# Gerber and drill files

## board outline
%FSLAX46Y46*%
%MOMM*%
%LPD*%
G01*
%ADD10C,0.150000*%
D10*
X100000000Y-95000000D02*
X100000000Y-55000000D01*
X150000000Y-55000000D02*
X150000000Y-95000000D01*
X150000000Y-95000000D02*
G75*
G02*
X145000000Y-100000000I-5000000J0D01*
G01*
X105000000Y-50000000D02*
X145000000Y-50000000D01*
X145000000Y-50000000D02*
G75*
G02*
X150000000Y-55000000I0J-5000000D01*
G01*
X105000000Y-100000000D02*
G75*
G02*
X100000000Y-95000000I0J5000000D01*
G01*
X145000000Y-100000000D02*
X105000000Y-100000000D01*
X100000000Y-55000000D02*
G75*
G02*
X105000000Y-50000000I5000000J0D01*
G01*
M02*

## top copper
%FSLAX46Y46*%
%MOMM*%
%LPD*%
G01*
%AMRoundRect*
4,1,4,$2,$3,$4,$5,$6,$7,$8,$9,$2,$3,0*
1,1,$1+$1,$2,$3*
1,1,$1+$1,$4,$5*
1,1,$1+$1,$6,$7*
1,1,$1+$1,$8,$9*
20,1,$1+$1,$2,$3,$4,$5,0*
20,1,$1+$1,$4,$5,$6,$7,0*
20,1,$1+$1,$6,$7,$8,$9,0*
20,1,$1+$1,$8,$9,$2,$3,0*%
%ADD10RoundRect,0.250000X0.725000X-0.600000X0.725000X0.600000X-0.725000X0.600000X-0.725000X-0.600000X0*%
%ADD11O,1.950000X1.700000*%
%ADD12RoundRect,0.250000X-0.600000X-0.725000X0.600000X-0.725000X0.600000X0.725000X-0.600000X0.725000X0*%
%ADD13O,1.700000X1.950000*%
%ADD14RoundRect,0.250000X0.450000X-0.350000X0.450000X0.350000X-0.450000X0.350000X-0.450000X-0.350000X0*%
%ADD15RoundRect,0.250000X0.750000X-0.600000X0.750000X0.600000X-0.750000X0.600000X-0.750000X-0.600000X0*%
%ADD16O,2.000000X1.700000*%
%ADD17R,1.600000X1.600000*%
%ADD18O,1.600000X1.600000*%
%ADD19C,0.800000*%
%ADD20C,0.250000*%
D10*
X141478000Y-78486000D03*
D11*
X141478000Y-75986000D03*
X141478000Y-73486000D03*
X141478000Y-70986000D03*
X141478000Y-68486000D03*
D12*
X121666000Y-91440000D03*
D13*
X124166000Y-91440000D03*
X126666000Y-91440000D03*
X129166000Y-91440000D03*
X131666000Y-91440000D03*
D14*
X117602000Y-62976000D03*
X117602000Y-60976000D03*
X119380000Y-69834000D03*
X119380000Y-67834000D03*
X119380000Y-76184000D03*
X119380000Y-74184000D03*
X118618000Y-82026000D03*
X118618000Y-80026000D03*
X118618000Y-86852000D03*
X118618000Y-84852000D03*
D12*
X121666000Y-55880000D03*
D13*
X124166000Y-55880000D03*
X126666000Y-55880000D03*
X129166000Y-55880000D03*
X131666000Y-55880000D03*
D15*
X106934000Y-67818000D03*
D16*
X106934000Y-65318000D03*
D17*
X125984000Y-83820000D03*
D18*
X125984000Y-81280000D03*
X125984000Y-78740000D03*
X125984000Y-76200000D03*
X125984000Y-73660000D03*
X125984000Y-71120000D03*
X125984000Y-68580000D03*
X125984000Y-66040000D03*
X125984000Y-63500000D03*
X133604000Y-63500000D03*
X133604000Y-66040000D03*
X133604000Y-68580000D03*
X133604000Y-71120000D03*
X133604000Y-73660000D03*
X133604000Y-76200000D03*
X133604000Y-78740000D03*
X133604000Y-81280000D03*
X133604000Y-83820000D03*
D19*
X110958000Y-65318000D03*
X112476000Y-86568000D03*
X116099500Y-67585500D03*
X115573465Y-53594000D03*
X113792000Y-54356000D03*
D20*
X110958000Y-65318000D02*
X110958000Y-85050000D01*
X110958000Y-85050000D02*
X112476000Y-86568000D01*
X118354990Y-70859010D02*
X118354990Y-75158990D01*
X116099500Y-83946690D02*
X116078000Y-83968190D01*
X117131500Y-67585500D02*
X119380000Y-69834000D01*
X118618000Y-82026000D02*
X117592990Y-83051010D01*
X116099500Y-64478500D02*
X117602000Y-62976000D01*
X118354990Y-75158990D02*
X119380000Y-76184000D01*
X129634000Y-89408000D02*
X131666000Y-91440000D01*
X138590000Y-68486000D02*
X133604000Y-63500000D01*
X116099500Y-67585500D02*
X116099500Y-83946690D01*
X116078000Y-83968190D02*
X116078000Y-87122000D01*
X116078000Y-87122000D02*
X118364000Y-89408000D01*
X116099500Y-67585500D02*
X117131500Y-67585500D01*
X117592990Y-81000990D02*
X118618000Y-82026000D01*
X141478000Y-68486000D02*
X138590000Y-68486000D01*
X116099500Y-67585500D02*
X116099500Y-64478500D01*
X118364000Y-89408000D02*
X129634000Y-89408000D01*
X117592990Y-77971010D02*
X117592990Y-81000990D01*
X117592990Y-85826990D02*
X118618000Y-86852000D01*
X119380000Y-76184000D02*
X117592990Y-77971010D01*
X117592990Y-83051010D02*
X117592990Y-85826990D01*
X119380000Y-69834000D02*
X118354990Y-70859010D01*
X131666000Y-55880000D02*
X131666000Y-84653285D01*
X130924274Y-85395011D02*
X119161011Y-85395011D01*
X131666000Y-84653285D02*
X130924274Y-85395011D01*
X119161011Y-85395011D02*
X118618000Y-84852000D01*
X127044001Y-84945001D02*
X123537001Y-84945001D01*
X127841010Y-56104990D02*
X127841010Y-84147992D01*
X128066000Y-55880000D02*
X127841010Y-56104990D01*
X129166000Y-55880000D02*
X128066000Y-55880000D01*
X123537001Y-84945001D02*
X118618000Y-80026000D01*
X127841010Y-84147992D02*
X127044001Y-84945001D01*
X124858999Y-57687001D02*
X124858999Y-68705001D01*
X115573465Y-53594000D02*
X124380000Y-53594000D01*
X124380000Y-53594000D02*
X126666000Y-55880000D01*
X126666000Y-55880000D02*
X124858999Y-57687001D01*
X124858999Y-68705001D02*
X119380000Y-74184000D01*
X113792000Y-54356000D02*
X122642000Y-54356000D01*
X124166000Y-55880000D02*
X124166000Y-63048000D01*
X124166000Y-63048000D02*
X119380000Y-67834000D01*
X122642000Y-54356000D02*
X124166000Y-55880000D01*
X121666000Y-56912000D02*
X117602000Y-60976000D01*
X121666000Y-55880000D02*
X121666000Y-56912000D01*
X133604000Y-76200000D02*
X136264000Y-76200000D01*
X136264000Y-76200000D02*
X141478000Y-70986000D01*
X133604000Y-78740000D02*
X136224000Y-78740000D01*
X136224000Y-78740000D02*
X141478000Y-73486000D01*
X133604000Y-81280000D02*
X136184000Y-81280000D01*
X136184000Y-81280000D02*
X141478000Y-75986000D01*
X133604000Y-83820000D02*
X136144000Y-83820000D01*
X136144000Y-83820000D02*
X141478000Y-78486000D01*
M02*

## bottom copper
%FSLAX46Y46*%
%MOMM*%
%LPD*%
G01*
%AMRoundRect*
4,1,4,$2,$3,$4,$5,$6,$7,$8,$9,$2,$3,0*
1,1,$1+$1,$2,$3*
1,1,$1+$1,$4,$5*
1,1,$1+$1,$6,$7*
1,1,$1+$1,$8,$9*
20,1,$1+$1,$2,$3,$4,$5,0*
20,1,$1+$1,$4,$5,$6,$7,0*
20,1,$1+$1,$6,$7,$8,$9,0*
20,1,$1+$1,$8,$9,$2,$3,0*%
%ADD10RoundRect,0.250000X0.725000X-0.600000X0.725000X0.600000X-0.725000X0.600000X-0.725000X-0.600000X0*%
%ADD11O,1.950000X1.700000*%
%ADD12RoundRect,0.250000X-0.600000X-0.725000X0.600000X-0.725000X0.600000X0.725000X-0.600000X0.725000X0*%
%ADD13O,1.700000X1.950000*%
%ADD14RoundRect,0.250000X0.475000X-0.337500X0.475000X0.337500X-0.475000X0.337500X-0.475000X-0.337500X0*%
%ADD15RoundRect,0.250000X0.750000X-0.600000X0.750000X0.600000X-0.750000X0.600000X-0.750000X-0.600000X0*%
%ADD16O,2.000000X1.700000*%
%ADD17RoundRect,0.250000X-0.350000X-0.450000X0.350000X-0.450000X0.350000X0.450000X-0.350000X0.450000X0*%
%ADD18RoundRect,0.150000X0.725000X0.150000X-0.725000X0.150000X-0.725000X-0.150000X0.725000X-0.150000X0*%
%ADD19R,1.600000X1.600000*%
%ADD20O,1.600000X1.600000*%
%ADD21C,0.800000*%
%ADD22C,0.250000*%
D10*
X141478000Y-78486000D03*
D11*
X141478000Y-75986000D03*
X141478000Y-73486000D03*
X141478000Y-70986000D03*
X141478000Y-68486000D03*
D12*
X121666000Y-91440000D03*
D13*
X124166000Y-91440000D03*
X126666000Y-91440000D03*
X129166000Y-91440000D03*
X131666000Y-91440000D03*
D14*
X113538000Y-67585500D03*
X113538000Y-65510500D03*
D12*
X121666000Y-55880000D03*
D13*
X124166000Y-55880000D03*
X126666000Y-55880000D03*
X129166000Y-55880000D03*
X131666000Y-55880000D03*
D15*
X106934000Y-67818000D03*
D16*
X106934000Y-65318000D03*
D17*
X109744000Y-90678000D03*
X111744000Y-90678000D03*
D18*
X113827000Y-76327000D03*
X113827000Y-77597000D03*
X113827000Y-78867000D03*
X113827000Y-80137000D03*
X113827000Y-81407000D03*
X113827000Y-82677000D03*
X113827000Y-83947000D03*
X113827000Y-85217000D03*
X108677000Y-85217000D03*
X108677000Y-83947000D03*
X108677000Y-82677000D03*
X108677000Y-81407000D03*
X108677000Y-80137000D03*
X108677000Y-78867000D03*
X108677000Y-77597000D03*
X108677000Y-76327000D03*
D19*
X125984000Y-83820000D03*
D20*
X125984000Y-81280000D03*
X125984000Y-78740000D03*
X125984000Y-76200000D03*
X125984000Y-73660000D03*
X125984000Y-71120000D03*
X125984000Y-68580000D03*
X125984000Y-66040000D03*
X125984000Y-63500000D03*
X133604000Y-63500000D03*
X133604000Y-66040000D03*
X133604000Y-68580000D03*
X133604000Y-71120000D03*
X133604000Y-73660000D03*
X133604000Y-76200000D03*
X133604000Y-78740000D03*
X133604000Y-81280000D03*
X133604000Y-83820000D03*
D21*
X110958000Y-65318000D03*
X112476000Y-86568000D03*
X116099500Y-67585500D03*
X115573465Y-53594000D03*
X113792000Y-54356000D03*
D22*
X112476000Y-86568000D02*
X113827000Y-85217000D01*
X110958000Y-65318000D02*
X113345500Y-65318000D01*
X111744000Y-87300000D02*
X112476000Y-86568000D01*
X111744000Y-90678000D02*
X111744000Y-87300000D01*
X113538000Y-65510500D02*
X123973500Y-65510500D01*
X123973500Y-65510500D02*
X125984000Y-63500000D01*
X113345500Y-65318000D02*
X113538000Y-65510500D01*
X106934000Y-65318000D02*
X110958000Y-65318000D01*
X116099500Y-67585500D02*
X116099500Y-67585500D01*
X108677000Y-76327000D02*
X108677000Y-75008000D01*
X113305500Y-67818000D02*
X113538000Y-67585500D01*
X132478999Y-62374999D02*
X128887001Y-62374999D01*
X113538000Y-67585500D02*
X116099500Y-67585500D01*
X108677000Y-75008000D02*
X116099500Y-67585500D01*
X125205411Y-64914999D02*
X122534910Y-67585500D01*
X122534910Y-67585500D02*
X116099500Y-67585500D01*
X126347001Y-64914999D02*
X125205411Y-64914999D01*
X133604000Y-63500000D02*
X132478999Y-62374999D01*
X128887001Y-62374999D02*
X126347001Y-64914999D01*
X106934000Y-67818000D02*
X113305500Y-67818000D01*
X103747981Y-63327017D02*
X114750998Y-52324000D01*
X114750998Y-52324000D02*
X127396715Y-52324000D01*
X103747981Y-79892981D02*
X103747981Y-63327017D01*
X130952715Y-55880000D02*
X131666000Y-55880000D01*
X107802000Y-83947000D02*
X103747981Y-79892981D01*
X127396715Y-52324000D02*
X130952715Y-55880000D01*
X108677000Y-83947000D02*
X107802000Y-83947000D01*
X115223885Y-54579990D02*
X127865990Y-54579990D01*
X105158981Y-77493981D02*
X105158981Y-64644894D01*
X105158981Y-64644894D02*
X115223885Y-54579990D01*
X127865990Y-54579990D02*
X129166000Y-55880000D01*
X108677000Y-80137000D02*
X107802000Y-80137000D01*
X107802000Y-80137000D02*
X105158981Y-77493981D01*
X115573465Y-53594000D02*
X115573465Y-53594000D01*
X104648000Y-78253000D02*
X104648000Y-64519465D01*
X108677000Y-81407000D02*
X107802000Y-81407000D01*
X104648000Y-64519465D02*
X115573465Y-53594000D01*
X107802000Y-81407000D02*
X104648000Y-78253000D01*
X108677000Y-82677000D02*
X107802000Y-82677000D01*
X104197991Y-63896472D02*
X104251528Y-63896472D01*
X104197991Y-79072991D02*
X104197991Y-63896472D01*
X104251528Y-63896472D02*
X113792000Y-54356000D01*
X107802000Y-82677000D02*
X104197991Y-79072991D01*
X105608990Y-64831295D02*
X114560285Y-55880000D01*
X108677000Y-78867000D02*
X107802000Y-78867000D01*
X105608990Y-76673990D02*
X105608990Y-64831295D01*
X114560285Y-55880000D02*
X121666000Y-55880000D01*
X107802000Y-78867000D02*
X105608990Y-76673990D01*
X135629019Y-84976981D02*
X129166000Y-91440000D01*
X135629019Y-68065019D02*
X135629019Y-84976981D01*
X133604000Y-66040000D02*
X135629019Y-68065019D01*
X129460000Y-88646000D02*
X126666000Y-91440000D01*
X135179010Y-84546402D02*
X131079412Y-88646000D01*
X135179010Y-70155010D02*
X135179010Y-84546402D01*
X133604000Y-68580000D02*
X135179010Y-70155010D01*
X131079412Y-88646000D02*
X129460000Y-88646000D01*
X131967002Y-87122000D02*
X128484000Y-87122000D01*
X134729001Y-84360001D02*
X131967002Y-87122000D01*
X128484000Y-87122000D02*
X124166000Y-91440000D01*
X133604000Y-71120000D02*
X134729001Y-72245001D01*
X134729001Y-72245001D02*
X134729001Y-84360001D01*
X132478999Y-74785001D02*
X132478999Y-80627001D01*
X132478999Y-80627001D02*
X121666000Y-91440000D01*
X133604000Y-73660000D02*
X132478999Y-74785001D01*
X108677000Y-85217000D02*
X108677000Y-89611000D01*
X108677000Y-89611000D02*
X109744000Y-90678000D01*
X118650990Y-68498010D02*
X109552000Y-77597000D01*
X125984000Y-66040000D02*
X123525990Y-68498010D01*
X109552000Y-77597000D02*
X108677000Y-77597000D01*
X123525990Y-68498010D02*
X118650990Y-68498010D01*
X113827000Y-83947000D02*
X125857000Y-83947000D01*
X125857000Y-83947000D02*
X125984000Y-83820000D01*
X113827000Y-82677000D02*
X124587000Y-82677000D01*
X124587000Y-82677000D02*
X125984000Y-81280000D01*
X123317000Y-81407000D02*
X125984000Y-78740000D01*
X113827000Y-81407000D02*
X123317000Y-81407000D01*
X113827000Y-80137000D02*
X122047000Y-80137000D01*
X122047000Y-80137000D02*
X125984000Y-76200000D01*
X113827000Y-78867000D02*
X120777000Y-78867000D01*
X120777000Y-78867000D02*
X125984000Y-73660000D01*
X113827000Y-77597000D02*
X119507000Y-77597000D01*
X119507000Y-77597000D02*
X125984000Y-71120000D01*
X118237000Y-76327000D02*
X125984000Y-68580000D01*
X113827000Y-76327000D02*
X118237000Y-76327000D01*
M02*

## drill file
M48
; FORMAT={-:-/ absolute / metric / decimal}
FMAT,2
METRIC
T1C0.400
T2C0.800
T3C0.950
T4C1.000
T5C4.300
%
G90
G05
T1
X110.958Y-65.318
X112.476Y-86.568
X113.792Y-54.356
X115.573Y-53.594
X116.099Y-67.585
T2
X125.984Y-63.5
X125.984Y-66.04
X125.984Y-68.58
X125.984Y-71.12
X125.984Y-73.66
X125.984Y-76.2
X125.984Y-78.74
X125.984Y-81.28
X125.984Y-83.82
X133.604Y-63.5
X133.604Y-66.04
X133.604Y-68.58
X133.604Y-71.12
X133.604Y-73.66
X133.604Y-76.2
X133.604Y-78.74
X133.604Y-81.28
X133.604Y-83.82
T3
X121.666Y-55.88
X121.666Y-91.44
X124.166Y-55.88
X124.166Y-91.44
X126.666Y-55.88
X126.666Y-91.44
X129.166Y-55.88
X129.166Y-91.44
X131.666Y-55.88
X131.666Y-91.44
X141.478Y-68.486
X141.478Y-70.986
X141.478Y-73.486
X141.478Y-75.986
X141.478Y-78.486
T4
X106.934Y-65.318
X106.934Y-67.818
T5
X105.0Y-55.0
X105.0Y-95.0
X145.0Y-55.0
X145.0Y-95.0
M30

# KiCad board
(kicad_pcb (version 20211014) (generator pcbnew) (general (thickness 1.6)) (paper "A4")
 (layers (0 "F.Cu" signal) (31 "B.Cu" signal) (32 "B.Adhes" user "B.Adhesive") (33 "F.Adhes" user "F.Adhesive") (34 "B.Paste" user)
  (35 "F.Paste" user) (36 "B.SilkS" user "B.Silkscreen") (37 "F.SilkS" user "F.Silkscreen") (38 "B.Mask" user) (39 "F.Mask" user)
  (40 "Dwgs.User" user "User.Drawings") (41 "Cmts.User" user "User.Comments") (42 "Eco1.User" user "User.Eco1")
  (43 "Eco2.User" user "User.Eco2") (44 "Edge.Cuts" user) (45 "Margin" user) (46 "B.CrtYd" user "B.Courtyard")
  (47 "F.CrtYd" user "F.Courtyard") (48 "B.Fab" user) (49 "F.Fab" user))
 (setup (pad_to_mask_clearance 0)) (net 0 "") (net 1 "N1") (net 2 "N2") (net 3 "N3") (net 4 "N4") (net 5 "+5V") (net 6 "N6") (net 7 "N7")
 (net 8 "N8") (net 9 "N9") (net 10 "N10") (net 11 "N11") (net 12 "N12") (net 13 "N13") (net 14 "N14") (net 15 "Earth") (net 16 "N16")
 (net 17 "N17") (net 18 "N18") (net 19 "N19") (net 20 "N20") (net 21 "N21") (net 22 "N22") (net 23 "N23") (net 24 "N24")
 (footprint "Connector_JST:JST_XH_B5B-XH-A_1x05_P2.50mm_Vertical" (layer "F.Cu") (at 141.478 78.486 90)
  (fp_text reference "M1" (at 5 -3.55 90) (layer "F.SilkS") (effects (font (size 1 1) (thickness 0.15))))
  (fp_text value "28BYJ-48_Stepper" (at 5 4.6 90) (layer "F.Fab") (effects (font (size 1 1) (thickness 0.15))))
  (pad "1" thru_hole roundrect locked (at 0 0 90) (size 1.7 1.95) (drill 0.95) (layers *.Cu *.Mask) (roundrect_rratio 0.147059) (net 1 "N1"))
  (pad "2" thru_hole oval locked (at 2.5 0 90) (size 1.7 1.95) (drill 0.95) (layers *.Cu *.Mask) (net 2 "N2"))
  (pad "3" thru_hole oval locked (at 5 0 90) (size 1.7 1.95) (drill 0.95) (layers *.Cu *.Mask) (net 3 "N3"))
  (pad "4" thru_hole oval locked (at 7.5 0 90) (size 1.7 1.95) (drill 0.95) (layers *.Cu *.Mask) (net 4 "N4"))
  (pad "5" thru_hole oval locked (at 10 0 90) (size 1.7 1.95) (drill 0.95) (layers *.Cu *.Mask) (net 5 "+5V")))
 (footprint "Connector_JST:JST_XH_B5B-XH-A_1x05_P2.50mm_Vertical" (layer "F.Cu") (at 121.666 91.44)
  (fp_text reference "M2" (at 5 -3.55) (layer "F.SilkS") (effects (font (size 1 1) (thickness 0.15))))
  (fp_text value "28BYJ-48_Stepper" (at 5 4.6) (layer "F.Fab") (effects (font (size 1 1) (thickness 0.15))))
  (pad "1" thru_hole roundrect locked (at 0 0) (size 1.7 1.95) (drill 0.95) (layers *.Cu *.Mask) (roundrect_rratio 0.147059) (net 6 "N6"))
  (pad "2" thru_hole oval locked (at 2.5 0) (size 1.7 1.95) (drill 0.95) (layers *.Cu *.Mask) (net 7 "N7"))
  (pad "3" thru_hole oval locked (at 5 0) (size 1.7 1.95) (drill 0.95) (layers *.Cu *.Mask) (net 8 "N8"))
  (pad "4" thru_hole oval locked (at 7.5 0) (size 1.7 1.95) (drill 0.95) (layers *.Cu *.Mask) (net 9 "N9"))
  (pad "5" thru_hole oval locked (at 10 0) (size 1.7 1.95) (drill 0.95) (layers *.Cu *.Mask) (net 5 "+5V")))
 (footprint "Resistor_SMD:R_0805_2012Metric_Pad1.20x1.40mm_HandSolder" (layer "F.Cu") (at 117.602 61.976 90)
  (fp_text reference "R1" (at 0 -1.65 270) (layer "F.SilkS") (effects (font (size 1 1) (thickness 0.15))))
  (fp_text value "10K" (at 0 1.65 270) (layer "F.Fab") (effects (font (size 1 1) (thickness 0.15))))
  (pad "1" smd roundrect locked (at -1 0 90) (size 1.2 1.4) (layers "F.Cu" "F.Paste" "F.Mask") (roundrect_rratio 0.208333) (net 5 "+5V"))
  (pad "2" smd roundrect locked (at 1 0 90) (size 1.2 1.4) (layers "F.Cu" "F.Paste" "F.Mask") (roundrect_rratio 0.208333) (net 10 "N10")))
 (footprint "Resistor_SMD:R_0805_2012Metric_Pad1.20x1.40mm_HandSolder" (layer "F.Cu") (at 119.38 68.834 90)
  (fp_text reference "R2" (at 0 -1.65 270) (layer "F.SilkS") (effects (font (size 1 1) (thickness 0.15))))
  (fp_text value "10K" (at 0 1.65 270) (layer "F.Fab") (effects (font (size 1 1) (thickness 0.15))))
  (pad "1" smd roundrect locked (at -1 0 90) (size 1.2 1.4) (layers "F.Cu" "F.Paste" "F.Mask") (roundrect_rratio 0.208333) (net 5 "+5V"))
  (pad "2" smd roundrect locked (at 1 0 90) (size 1.2 1.4) (layers "F.Cu" "F.Paste" "F.Mask") (roundrect_rratio 0.208333) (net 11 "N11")))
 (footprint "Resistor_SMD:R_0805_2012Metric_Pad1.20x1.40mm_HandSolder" (layer "F.Cu") (at 119.38 75.184 90)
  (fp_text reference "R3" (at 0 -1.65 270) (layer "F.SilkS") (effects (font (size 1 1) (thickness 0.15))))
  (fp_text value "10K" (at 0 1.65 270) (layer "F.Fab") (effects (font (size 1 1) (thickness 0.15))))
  (pad "1" smd roundrect locked (at -1 0 90) (size 1.2 1.4) (layers "F.Cu" "F.Paste" "F.Mask") (roundrect_rratio 0.208333) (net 5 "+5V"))
  (pad "2" smd roundrect locked (at 1 0 90) (size 1.2 1.4) (layers "F.Cu" "F.Paste" "F.Mask") (roundrect_rratio 0.208333) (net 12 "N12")))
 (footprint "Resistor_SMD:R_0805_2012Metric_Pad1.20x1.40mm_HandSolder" (layer "F.Cu") (at 118.618 81.026 90)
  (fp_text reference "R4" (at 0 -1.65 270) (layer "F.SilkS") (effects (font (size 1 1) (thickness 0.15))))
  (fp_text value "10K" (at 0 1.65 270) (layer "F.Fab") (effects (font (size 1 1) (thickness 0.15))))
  (pad "1" smd roundrect locked (at -1 0 90) (size 1.2 1.4) (layers "F.Cu" "F.Paste" "F.Mask") (roundrect_rratio 0.208333) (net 5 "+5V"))
  (pad "2" smd roundrect locked (at 1 0 90) (size 1.2 1.4) (layers "F.Cu" "F.Paste" "F.Mask") (roundrect_rratio 0.208333) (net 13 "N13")))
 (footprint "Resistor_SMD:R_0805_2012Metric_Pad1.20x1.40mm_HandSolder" (layer "F.Cu") (at 118.618 85.852 90)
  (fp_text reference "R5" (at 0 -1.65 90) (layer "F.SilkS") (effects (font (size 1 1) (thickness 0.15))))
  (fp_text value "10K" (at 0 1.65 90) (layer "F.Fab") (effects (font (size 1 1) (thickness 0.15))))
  (pad "1" smd roundrect locked (at -1 0 90) (size 1.2 1.4) (layers "F.Cu" "F.Paste" "F.Mask") (roundrect_rratio 0.208333) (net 5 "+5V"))
  (pad "2" smd roundrect locked (at 1 0 90) (size 1.2 1.4) (layers "F.Cu" "F.Paste" "F.Mask") (roundrect_rratio 0.208333) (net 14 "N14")))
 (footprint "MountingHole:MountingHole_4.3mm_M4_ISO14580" (layer "F.Cu") (at 105 55)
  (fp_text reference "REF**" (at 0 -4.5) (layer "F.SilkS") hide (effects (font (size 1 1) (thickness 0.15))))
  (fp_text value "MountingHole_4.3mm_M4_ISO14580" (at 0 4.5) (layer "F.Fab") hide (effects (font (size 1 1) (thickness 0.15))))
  (pad "" np_thru_hole circle locked (at 0 0) (size 4.3 4.3) (drill 4.3) (layers *.Cu *.Mask)))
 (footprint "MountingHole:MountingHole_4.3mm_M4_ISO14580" (layer "F.Cu") (at 145 55)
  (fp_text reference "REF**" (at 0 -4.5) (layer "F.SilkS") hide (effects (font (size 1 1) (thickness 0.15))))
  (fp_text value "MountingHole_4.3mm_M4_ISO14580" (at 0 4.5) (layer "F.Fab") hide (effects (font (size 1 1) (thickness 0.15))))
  (pad "" np_thru_hole circle locked (at 0 0) (size 4.3 4.3) (drill 4.3) (layers *.Cu *.Mask)))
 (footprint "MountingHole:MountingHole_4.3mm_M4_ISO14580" (layer "F.Cu") (at 105 95)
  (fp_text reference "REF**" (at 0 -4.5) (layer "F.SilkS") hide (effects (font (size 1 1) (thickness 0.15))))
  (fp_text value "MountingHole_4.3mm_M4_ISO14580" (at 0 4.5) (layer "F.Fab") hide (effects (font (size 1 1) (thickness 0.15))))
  (pad "" np_thru_hole circle locked (at 0 0) (size 4.3 4.3) (drill 4.3) (layers *.Cu *.Mask)))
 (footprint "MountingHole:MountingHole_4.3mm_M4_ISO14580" (layer "F.Cu") (at 145 95)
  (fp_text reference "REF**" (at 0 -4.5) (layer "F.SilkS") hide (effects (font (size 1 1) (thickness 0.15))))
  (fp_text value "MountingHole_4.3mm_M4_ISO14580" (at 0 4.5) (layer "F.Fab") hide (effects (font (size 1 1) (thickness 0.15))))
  (pad "" np_thru_hole circle locked (at 0 0) (size 4.3 4.3) (drill 4.3) (layers *.Cu *.Mask)))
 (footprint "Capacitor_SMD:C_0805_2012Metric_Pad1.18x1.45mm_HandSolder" (layer "B.Cu") (at 113.538 66.548 90)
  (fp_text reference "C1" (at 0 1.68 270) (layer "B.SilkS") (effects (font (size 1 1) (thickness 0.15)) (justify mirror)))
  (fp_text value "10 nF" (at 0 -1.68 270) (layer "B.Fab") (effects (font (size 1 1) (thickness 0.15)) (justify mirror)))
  (pad "1" smd roundrect locked (at -1.0375 0 90) (size 1.175 1.45) (layers "B.Cu" "B.Paste" "B.Mask") (roundrect_rratio 0.212766)
   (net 5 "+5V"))
  (pad "2" smd roundrect locked (at 1.0375 0 90) (size 1.175 1.45) (layers "B.Cu" "B.Paste" "B.Mask") (roundrect_rratio 0.212766)
   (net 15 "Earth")))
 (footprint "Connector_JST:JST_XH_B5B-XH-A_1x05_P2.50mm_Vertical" (layer "B.Cu") (at 121.666 55.88)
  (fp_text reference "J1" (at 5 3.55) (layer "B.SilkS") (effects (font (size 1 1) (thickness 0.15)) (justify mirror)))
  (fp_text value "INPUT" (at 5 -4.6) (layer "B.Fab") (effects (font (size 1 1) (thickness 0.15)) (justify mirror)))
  (pad "1" thru_hole roundrect locked (at 0 0) (size 1.7 1.95) (drill 0.95) (layers *.Cu *.Mask) (roundrect_rratio 0.147059) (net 10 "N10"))
  (pad "2" thru_hole oval locked (at 2.5 0) (size 1.7 1.95) (drill 0.95) (layers *.Cu *.Mask) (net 11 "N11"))
  (pad "3" thru_hole oval locked (at 5 0) (size 1.7 1.95) (drill 0.95) (layers *.Cu *.Mask) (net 12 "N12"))
  (pad "4" thru_hole oval locked (at 7.5 0) (size 1.7 1.95) (drill 0.95) (layers *.Cu *.Mask) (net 13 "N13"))
  (pad "5" thru_hole oval locked (at 10 0) (size 1.7 1.95) (drill 0.95) (layers *.Cu *.Mask) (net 14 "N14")))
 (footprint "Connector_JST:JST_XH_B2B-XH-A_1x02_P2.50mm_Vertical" (layer "B.Cu") (at 106.934 67.818 90)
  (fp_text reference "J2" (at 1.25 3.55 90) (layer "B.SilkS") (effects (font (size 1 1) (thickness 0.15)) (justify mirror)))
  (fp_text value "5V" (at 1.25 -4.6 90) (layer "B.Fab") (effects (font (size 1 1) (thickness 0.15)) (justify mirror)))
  (pad "1" thru_hole roundrect locked (at 0 0 90) (size 1.7 2) (drill 1) (layers *.Cu *.Mask) (roundrect_rratio 0.147059) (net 5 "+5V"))
  (pad "2" thru_hole oval locked (at 2.5 0 90) (size 1.7 2) (drill 1) (layers *.Cu *.Mask) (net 15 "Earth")))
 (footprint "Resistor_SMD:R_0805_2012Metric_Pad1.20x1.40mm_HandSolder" (layer "B.Cu") (at 110.744 90.678)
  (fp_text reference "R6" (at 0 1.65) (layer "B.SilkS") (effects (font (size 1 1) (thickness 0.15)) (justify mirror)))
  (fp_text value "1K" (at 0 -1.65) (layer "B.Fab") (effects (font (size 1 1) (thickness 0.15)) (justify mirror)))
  (pad "1" smd roundrect locked (at -1 0) (size 1.2 1.4) (layers "B.Cu" "B.Paste" "B.Mask") (roundrect_rratio 0.208333) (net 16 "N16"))
  (pad "2" smd roundrect locked (at 1 0) (size 1.2 1.4) (layers "B.Cu" "B.Paste" "B.Mask") (roundrect_rratio 0.208333) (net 15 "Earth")))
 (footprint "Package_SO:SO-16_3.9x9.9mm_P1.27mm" (layer "B.Cu") (at 111.252 80.772 180)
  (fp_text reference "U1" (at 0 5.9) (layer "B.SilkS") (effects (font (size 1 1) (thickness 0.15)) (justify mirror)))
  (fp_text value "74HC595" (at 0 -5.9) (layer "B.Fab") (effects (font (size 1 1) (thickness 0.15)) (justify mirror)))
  (pad "1" smd roundrect locked (at -2.575 4.445 180) (size 1.75 0.6) (layers "B.Cu" "B.Paste" "B.Mask") (roundrect_rratio 0.25)
   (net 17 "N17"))
  (pad "2" smd roundrect locked (at -2.575 3.175 180) (size 1.75 0.6) (layers "B.Cu" "B.Paste" "B.Mask") (roundrect_rratio 0.25)
   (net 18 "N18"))
  (pad "3" smd roundrect locked (at -2.575 1.905 180) (size 1.75 0.6) (layers "B.Cu" "B.Paste" "B.Mask") (roundrect_rratio 0.25)
   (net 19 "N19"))
  (pad "4" smd roundrect locked (at -2.575 0.635 180) (size 1.75 0.6) (layers "B.Cu" "B.Paste" "B.Mask") (roundrect_rratio 0.25)
   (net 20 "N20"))
  (pad "5" smd roundrect locked (at -2.575 -0.635 180) (size 1.75 0.6) (layers "B.Cu" "B.Paste" "B.Mask") (roundrect_rratio 0.25)
   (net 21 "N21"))
  (pad "6" smd roundrect locked (at -2.575 -1.905 180) (size 1.75 0.6) (layers "B.Cu" "B.Paste" "B.Mask") (roundrect_rratio 0.25)
   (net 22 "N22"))
  (pad "7" smd roundrect locked (at -2.575 -3.175 180) (size 1.75 0.6) (layers "B.Cu" "B.Paste" "B.Mask") (roundrect_rratio 0.25)
   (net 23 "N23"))
  (pad "8" smd roundrect locked (at -2.575 -4.445 180) (size 1.75 0.6) (layers "B.Cu" "B.Paste" "B.Mask") (roundrect_rratio 0.25)
   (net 15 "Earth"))
  (pad "9" smd roundrect locked (at 2.575 -4.445 180) (size 1.75 0.6) (layers "B.Cu" "B.Paste" "B.Mask") (roundrect_rratio 0.25)
   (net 16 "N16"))
  (pad "10" smd roundrect locked (at 2.575 -3.175 180) (size 1.75 0.6) (layers "B.Cu" "B.Paste" "B.Mask") (roundrect_rratio 0.25)
   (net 14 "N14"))
  (pad "11" smd roundrect locked (at 2.575 -1.905 180) (size 1.75 0.6) (layers "B.Cu" "B.Paste" "B.Mask") (roundrect_rratio 0.25)
   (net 11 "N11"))
  (pad "12" smd roundrect locked (at 2.575 -0.635 180) (size 1.75 0.6) (layers "B.Cu" "B.Paste" "B.Mask") (roundrect_rratio 0.25)
   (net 12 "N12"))
  (pad "13" smd roundrect locked (at 2.575 0.635 180) (size 1.75 0.6) (layers "B.Cu" "B.Paste" "B.Mask") (roundrect_rratio 0.25)
   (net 13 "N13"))
  (pad "14" smd roundrect locked (at 2.575 1.905 180) (size 1.75 0.6) (layers "B.Cu" "B.Paste" "B.Mask") (roundrect_rratio 0.25)
   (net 10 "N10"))
  (pad "15" smd roundrect locked (at 2.575 3.175 180) (size 1.75 0.6) (layers "B.Cu" "B.Paste" "B.Mask") (roundrect_rratio 0.25)
   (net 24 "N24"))
  (pad "16" smd roundrect locked (at 2.575 4.445 180) (size 1.75 0.6) (layers "B.Cu" "B.Paste" "B.Mask") (roundrect_rratio 0.25)
   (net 5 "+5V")))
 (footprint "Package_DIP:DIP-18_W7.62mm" (layer "B.Cu") (at 125.984 83.82)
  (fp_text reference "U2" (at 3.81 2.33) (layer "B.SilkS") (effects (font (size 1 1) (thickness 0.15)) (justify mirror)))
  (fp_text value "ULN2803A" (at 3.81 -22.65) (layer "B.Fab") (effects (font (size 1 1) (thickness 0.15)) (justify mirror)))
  (pad "1" thru_hole rect locked (at 0 0) (size 1.6 1.6) (drill 0.8) (layers *.Cu *.Mask) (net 23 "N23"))
  (pad "2" thru_hole oval locked (at 0 -2.54) (size 1.6 1.6) (drill 0.8) (layers *.Cu *.Mask) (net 22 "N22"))
  (pad "3" thru_hole oval locked (at 0 -5.08) (size 1.6 1.6) (drill 0.8) (layers *.Cu *.Mask) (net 21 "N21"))
  (pad "4" thru_hole oval locked (at 0 -7.62) (size 1.6 1.6) (drill 0.8) (layers *.Cu *.Mask) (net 20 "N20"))
  (pad "5" thru_hole oval locked (at 0 -10.16) (size 1.6 1.6) (drill 0.8) (layers *.Cu *.Mask) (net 19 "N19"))
  (pad "6" thru_hole oval locked (at 0 -12.7) (size 1.6 1.6) (drill 0.8) (layers *.Cu *.Mask) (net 18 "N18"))
  (pad "7" thru_hole oval locked (at 0 -15.24) (size 1.6 1.6) (drill 0.8) (layers *.Cu *.Mask) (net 17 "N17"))
  (pad "8" thru_hole oval locked (at 0 -17.78) (size 1.6 1.6) (drill 0.8) (layers *.Cu *.Mask) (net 24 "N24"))
  (pad "9" thru_hole oval locked (at 0 -20.32) (size 1.6 1.6) (drill 0.8) (layers *.Cu *.Mask) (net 15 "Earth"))
  (pad "10" thru_hole oval locked (at 7.62 -20.32) (size 1.6 1.6) (drill 0.8) (layers *.Cu *.Mask) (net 5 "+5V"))
  (pad "11" thru_hole oval locked (at 7.62 -17.78) (size 1.6 1.6) (drill 0.8) (layers *.Cu *.Mask) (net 9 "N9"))
  (pad "12" thru_hole oval locked (at 7.62 -15.24) (size 1.6 1.6) (drill 0.8) (layers *.Cu *.Mask) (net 8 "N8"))
  (pad "13" thru_hole oval locked (at 7.62 -12.7) (size 1.6 1.6) (drill 0.8) (layers *.Cu *.Mask) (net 7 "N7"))
  (pad "14" thru_hole oval locked (at 7.62 -10.16) (size 1.6 1.6) (drill 0.8) (layers *.Cu *.Mask) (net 6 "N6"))
  (pad "15" thru_hole oval locked (at 7.62 -7.62) (size 1.6 1.6) (drill 0.8) (layers *.Cu *.Mask) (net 4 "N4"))
  (pad "16" thru_hole oval locked (at 7.62 -5.08) (size 1.6 1.6) (drill 0.8) (layers *.Cu *.Mask) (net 3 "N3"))
  (pad "17" thru_hole oval locked (at 7.62 -2.54) (size 1.6 1.6) (drill 0.8) (layers *.Cu *.Mask) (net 2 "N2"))
  (pad "18" thru_hole oval locked (at 7.62 0) (size 1.6 1.6) (drill 0.8) (layers *.Cu *.Mask) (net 1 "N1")))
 (gr_line (start 100 95) (end 100 55) (layer "Edge.Cuts") (width 0.15))
 (gr_line (start 150 55) (end 150 95) (layer "Edge.Cuts") (width 0.15))
 (gr_arc (start 150 95) (mid 148.535534 98.535534) (end 145 100) (layer "Edge.Cuts") (width 0.15))
 (gr_line (start 105 50) (end 145 50) (layer "Edge.Cuts") (width 0.15))
 (gr_arc (start 145 50) (mid 148.535534 51.464466) (end 150 55) (layer "Edge.Cuts") (width 0.15))
 (gr_arc (start 105 100) (mid 101.464466 98.535534) (end 100 95) (layer "Edge.Cuts") (width 0.15))
 (gr_line (start 145 100) (end 105 100) (layer "Edge.Cuts") (width 0.15))
 (gr_arc (start 100 55) (mid 101.464466 51.464466) (end 105 50) (layer "Edge.Cuts") (width 0.15))
 (segment (start 110.958 65.318) (end 110.958 85.05) (width 0.25) (layer "F.Cu") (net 15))
 (segment (start 110.958 85.05) (end 112.476 86.568) (width 0.25) (layer "F.Cu") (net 15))
 (via (at 110.958 65.318) (size 0.8) (drill 0.4) (layers "F.Cu" "B.Cu") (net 15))
 (via (at 112.476 86.568) (size 0.8) (drill 0.4) (layers "F.Cu" "B.Cu") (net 15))
 (segment (start 112.476 86.568) (end 113.827 85.217) (width 0.25) (layer "B.Cu") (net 15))
 (segment (start 110.958 65.318) (end 113.3455 65.318) (width 0.25) (layer "B.Cu") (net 15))
 (segment (start 111.744 87.3) (end 112.476 86.568) (width 0.25) (layer "B.Cu") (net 15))
 (segment (start 111.744 90.678) (end 111.744 87.3) (width 0.25) (layer "B.Cu") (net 15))
 (segment (start 113.538 65.5105) (end 123.9735 65.5105) (width 0.25) (layer "B.Cu") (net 15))
 (segment (start 123.9735 65.5105) (end 125.984 63.5) (width 0.25) (layer "B.Cu") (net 15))
 (segment (start 113.3455 65.318) (end 113.538 65.5105) (width 0.25) (layer "B.Cu") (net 15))
 (segment (start 106.934 65.318) (end 110.958 65.318) (width 0.25) (layer "B.Cu") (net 15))
 (segment (start 118.35499 70.85901) (end 118.35499 75.15899) (width 0.25) (layer "F.Cu") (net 5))
 (segment (start 116.0995 83.94669) (end 116.078 83.96819) (width 0.25) (layer "F.Cu") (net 5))
 (segment (start 117.1315 67.5855) (end 119.38 69.834) (width 0.25) (layer "F.Cu") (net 5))
 (segment (start 118.618 82.026) (end 117.59299 83.05101) (width 0.25) (layer "F.Cu") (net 5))
 (segment (start 116.0995 64.4785) (end 117.602 62.976) (width 0.25) (layer "F.Cu") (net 5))
 (segment (start 118.35499 75.15899) (end 119.38 76.184) (width 0.25) (layer "F.Cu") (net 5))
 (segment (start 129.634 89.408) (end 131.666 91.44) (width 0.25) (layer "F.Cu") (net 5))
 (segment (start 138.59 68.486) (end 133.604 63.5) (width 0.25) (layer "F.Cu") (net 5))
 (segment (start 116.0995 67.5855) (end 116.0995 83.94669) (width 0.25) (layer "F.Cu") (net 5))
 (segment (start 116.078 83.96819) (end 116.078 87.122) (width 0.25) (layer "F.Cu") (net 5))
 (segment (start 116.078 87.122) (end 118.364 89.408) (width 0.25) (layer "F.Cu") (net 5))
 (segment (start 116.0995 67.5855) (end 117.1315 67.5855) (width 0.25) (layer "F.Cu") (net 5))
 (segment (start 117.59299 81.00099) (end 118.618 82.026) (width 0.25) (layer "F.Cu") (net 5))
 (segment (start 141.478 68.486) (end 138.59 68.486) (width 0.25) (layer "F.Cu") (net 5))
 (segment (start 116.0995 67.5855) (end 116.0995 64.4785) (width 0.25) (layer "F.Cu") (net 5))
 (segment (start 118.364 89.408) (end 129.634 89.408) (width 0.25) (layer "F.Cu") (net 5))
 (segment (start 117.59299 77.97101) (end 117.59299 81.00099) (width 0.25) (layer "F.Cu") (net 5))
 (segment (start 117.59299 85.82699) (end 118.618 86.852) (width 0.25) (layer "F.Cu") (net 5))
 (segment (start 119.38 76.184) (end 117.59299 77.97101) (width 0.25) (layer "F.Cu") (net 5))
 (segment (start 117.59299 83.05101) (end 117.59299 85.82699) (width 0.25) (layer "F.Cu") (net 5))
 (segment (start 119.38 69.834) (end 118.35499 70.85901) (width 0.25) (layer "F.Cu") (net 5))
 (via (at 116.0995 67.5855) (size 0.8) (drill 0.4) (layers "F.Cu" "B.Cu") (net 5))
 (segment (start 116.0995 67.5855) (end 116.0995 67.5855) (width 0.25) (layer "B.Cu") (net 5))
 (segment (start 108.677 76.327) (end 108.677 75.008) (width 0.25) (layer "B.Cu") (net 5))
 (segment (start 113.3055 67.818) (end 113.538 67.5855) (width 0.25) (layer "B.Cu") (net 5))
 (segment (start 132.478999 62.374999) (end 128.887001 62.374999) (width 0.25) (layer "B.Cu") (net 5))
 (segment (start 113.538 67.5855) (end 116.0995 67.5855) (width 0.25) (layer "B.Cu") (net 5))
 (segment (start 108.677 75.008) (end 116.0995 67.5855) (width 0.25) (layer "B.Cu") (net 5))
 (segment (start 125.205411 64.914999) (end 122.53491 67.5855) (width 0.25) (layer "B.Cu") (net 5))
 (segment (start 122.53491 67.5855) (end 116.0995 67.5855) (width 0.25) (layer "B.Cu") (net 5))
 (segment (start 126.347001 64.914999) (end 125.205411 64.914999) (width 0.25) (layer "B.Cu") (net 5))
 (segment (start 133.604 63.5) (end 132.478999 62.374999) (width 0.25) (layer "B.Cu") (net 5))
 (segment (start 128.887001 62.374999) (end 126.347001 64.914999) (width 0.25) (layer "B.Cu") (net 5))
 (segment (start 106.934 67.818) (end 113.3055 67.818) (width 0.25) (layer "B.Cu") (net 5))
 (segment (start 131.666 55.88) (end 131.666 84.653285) (width 0.25) (layer "F.Cu") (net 14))
 (segment (start 130.924274 85.395011) (end 119.161011 85.395011) (width 0.25) (layer "F.Cu") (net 14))
 (segment (start 131.666 84.653285) (end 130.924274 85.395011) (width 0.25) (layer "F.Cu") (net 14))
 (segment (start 119.161011 85.395011) (end 118.618 84.852) (width 0.25) (layer "F.Cu") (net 14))
 (segment (start 103.747981 63.327017) (end 114.750998 52.324) (width 0.25) (layer "B.Cu") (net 14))
 (segment (start 114.750998 52.324) (end 127.396715 52.324) (width 0.25) (layer "B.Cu") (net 14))
 (segment (start 103.747981 79.892981) (end 103.747981 63.327017) (width 0.25) (layer "B.Cu") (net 14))
 (segment (start 130.952715 55.88) (end 131.666 55.88) (width 0.25) (layer "B.Cu") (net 14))
 (segment (start 107.802 83.947) (end 103.747981 79.892981) (width 0.25) (layer "B.Cu") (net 14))
 (segment (start 127.396715 52.324) (end 130.952715 55.88) (width 0.25) (layer "B.Cu") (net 14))
 (segment (start 108.677 83.947) (end 107.802 83.947) (width 0.25) (layer "B.Cu") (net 14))
 (segment (start 127.044001 84.945001) (end 123.537001 84.945001) (width 0.25) (layer "F.Cu") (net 13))
 (segment (start 127.84101 56.10499) (end 127.84101 84.147992) (width 0.25) (layer "F.Cu") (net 13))
 (segment (start 128.066 55.88) (end 127.84101 56.10499) (width 0.25) (layer "F.Cu") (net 13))
 (segment (start 129.166 55.88) (end 128.066 55.88) (width 0.25) (layer "F.Cu") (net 13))
 (segment (start 123.537001 84.945001) (end 118.618 80.026) (width 0.25) (layer "F.Cu") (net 13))
 (segment (start 127.84101 84.147992) (end 127.044001 84.945001) (width 0.25) (layer "F.Cu") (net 13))
 (segment (start 115.223885 54.57999) (end 127.86599 54.57999) (width 0.25) (layer "B.Cu") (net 13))
 (segment (start 105.158981 77.493981) (end 105.158981 64.644894) (width 0.25) (layer "B.Cu") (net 13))
 (segment (start 105.158981 64.644894) (end 115.223885 54.57999) (width 0.25) (layer "B.Cu") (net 13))
 (segment (start 127.86599 54.57999) (end 129.166 55.88) (width 0.25) (layer "B.Cu") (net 13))
 (segment (start 108.677 80.137) (end 107.802 80.137) (width 0.25) (layer "B.Cu") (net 13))
 (segment (start 107.802 80.137) (end 105.158981 77.493981) (width 0.25) (layer "B.Cu") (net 13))
 (segment (start 124.858999 57.687001) (end 124.858999 68.705001) (width 0.25) (layer "F.Cu") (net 12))
 (segment (start 115.573465 53.594) (end 124.38 53.594) (width 0.25) (layer "F.Cu") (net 12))
 (segment (start 124.38 53.594) (end 126.666 55.88) (width 0.25) (layer "F.Cu") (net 12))
 (segment (start 126.666 55.88) (end 124.858999 57.687001) (width 0.25) (layer "F.Cu") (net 12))
 (segment (start 124.858999 68.705001) (end 119.38 74.184) (width 0.25) (layer "F.Cu") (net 12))
 (via (at 115.573465 53.594) (size 0.8) (drill 0.4) (layers "F.Cu" "B.Cu") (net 12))
 (segment (start 115.573465 53.594) (end 115.573465 53.594) (width 0.25) (layer "B.Cu") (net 12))
 (segment (start 104.648 78.253) (end 104.648 64.519465) (width 0.25) (layer "B.Cu") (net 12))
 (segment (start 108.677 81.407) (end 107.802 81.407) (width 0.25) (layer "B.Cu") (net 12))
 (segment (start 104.648 64.519465) (end 115.573465 53.594) (width 0.25) (layer "B.Cu") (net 12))
 (segment (start 107.802 81.407) (end 104.648 78.253) (width 0.25) (layer "B.Cu") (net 12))
 (segment (start 113.792 54.356) (end 122.642 54.356) (width 0.25) (layer "F.Cu") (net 11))
 (segment (start 124.166 55.88) (end 124.166 63.048) (width 0.25) (layer "F.Cu") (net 11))
 (segment (start 124.166 63.048) (end 119.38 67.834) (width 0.25) (layer "F.Cu") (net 11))
 (segment (start 122.642 54.356) (end 124.166 55.88) (width 0.25) (layer "F.Cu") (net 11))
 (via (at 113.792 54.356) (size 0.8) (drill 0.4) (layers "F.Cu" "B.Cu") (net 11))
 (segment (start 108.677 82.677) (end 107.802 82.677) (width 0.25) (layer "B.Cu") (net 11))
 (segment (start 104.197991 63.896472) (end 104.251528 63.896472) (width 0.25) (layer "B.Cu") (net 11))
 (segment (start 104.197991 79.072991) (end 104.197991 63.896472) (width 0.25) (layer "B.Cu") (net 11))
 (segment (start 104.251528 63.896472) (end 113.792 54.356) (width 0.25) (layer "B.Cu") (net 11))
 (segment (start 107.802 82.677) (end 104.197991 79.072991) (width 0.25) (layer "B.Cu") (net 11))
 (segment (start 121.666 56.912) (end 117.602 60.976) (width 0.25) (layer "F.Cu") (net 10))
 (segment (start 121.666 55.88) (end 121.666 56.912) (width 0.25) (layer "F.Cu") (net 10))
 (segment (start 105.60899 64.831295) (end 114.560285 55.88) (width 0.25) (layer "B.Cu") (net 10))
 (segment (start 108.677 78.867) (end 107.802 78.867) (width 0.25) (layer "B.Cu") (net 10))
 (segment (start 105.60899 76.67399) (end 105.60899 64.831295) (width 0.25) (layer "B.Cu") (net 10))
 (segment (start 114.560285 55.88) (end 121.666 55.88) (width 0.25) (layer "B.Cu") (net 10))
 (segment (start 107.802 78.867) (end 105.60899 76.67399) (width 0.25) (layer "B.Cu") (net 10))
 (segment (start 133.604 76.2) (end 136.264 76.2) (width 0.25) (layer "F.Cu") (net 4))
 (segment (start 136.264 76.2) (end 141.478 70.986) (width 0.25) (layer "F.Cu") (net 4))
 (segment (start 133.604 78.74) (end 136.224 78.74) (width 0.25) (layer "F.Cu") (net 3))
 (segment (start 136.224 78.74) (end 141.478 73.486) (width 0.25) (layer "F.Cu") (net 3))
 (segment (start 133.604 81.28) (end 136.184 81.28) (width 0.25) (layer "F.Cu") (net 2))
 (segment (start 136.184 81.28) (end 141.478 75.986) (width 0.25) (layer "F.Cu") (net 2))
 (segment (start 133.604 83.82) (end 136.144 83.82) (width 0.25) (layer "F.Cu") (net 1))
 (segment (start 136.144 83.82) (end 141.478 78.486) (width 0.25) (layer "F.Cu") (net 1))
 (segment (start 135.629019 84.976981) (end 129.166 91.44) (width 0.25) (layer "B.Cu") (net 9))
 (segment (start 135.629019 68.065019) (end 135.629019 84.976981) (width 0.25) (layer "B.Cu") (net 9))
 (segment (start 133.604 66.04) (end 135.629019 68.065019) (width 0.25) (layer "B.Cu") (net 9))
 (segment (start 129.46 88.646) (end 126.666 91.44) (width 0.25) (layer "B.Cu") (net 8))
 (segment (start 135.17901 84.546402) (end 131.079412 88.646) (width 0.25) (layer "B.Cu") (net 8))
 (segment (start 135.17901 70.15501) (end 135.17901 84.546402) (width 0.25) (layer "B.Cu") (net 8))
 (segment (start 133.604 68.58) (end 135.17901 70.15501) (width 0.25) (layer "B.Cu") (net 8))
 (segment (start 131.079412 88.646) (end 129.46 88.646) (width 0.25) (layer "B.Cu") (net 8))
 (segment (start 131.967002 87.122) (end 128.484 87.122) (width 0.25) (layer "B.Cu") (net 7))
 (segment (start 134.729001 84.360001) (end 131.967002 87.122) (width 0.25) (layer "B.Cu") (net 7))
 (segment (start 128.484 87.122) (end 124.166 91.44) (width 0.25) (layer "B.Cu") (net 7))
 (segment (start 133.604 71.12) (end 134.729001 72.245001) (width 0.25) (layer "B.Cu") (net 7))
 (segment (start 134.729001 72.245001) (end 134.729001 84.360001) (width 0.25) (layer "B.Cu") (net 7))
 (segment (start 132.478999 74.785001) (end 132.478999 80.627001) (width 0.25) (layer "B.Cu") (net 6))
 (segment (start 132.478999 80.627001) (end 121.666 91.44) (width 0.25) (layer "B.Cu") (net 6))
 (segment (start 133.604 73.66) (end 132.478999 74.785001) (width 0.25) (layer "B.Cu") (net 6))
 (segment (start 108.677 85.217) (end 108.677 89.611) (width 0.25) (layer "B.Cu") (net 16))
 (segment (start 108.677 89.611) (end 109.744 90.678) (width 0.25) (layer "B.Cu") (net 16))
 (segment (start 118.65099 68.49801) (end 109.552 77.597) (width 0.25) (layer "B.Cu") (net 24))
 (segment (start 125.984 66.04) (end 123.52599 68.49801) (width 0.25) (layer "B.Cu") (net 24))
 (segment (start 109.552 77.597) (end 108.677 77.597) (width 0.25) (layer "B.Cu") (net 24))
 (segment (start 123.52599 68.49801) (end 118.65099 68.49801) (width 0.25) (layer "B.Cu") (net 24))
 (segment (start 113.827 83.947) (end 125.857 83.947) (width 0.25) (layer "B.Cu") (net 23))
 (segment (start 125.857 83.947) (end 125.984 83.82) (width 0.25) (layer "B.Cu") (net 23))
 (segment (start 113.827 82.677) (end 124.587 82.677) (width 0.25) (layer "B.Cu") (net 22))
 (segment (start 124.587 82.677) (end 125.984 81.28) (width 0.25) (layer "B.Cu") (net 22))
 (segment (start 123.317 81.407) (end 125.984 78.74) (width 0.25) (layer "B.Cu") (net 21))
 (segment (start 113.827 81.407) (end 123.317 81.407) (width 0.25) (layer "B.Cu") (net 21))
 (segment (start 113.827 80.137) (end 122.047 80.137) (width 0.25) (layer "B.Cu") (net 20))
 (segment (start 122.047 80.137) (end 125.984 76.2) (width 0.25) (layer "B.Cu") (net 20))
 (segment (start 113.827 78.867) (end 120.777 78.867) (width 0.25) (layer "B.Cu") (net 19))
 (segment (start 120.777 78.867) (end 125.984 73.66) (width 0.25) (layer "B.Cu") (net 19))
 (segment (start 113.827 77.597) (end 119.507 77.597) (width 0.25) (layer "B.Cu") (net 18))
 (segment (start 119.507 77.597) (end 125.984 71.12) (width 0.25) (layer "B.Cu") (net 18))
 (segment (start 118.237 76.327) (end 125.984 68.58) (width 0.25) (layer "B.Cu") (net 17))
 (segment (start 113.827 76.327) (end 118.237 76.327) (width 0.25) (layer "B.Cu") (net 17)))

